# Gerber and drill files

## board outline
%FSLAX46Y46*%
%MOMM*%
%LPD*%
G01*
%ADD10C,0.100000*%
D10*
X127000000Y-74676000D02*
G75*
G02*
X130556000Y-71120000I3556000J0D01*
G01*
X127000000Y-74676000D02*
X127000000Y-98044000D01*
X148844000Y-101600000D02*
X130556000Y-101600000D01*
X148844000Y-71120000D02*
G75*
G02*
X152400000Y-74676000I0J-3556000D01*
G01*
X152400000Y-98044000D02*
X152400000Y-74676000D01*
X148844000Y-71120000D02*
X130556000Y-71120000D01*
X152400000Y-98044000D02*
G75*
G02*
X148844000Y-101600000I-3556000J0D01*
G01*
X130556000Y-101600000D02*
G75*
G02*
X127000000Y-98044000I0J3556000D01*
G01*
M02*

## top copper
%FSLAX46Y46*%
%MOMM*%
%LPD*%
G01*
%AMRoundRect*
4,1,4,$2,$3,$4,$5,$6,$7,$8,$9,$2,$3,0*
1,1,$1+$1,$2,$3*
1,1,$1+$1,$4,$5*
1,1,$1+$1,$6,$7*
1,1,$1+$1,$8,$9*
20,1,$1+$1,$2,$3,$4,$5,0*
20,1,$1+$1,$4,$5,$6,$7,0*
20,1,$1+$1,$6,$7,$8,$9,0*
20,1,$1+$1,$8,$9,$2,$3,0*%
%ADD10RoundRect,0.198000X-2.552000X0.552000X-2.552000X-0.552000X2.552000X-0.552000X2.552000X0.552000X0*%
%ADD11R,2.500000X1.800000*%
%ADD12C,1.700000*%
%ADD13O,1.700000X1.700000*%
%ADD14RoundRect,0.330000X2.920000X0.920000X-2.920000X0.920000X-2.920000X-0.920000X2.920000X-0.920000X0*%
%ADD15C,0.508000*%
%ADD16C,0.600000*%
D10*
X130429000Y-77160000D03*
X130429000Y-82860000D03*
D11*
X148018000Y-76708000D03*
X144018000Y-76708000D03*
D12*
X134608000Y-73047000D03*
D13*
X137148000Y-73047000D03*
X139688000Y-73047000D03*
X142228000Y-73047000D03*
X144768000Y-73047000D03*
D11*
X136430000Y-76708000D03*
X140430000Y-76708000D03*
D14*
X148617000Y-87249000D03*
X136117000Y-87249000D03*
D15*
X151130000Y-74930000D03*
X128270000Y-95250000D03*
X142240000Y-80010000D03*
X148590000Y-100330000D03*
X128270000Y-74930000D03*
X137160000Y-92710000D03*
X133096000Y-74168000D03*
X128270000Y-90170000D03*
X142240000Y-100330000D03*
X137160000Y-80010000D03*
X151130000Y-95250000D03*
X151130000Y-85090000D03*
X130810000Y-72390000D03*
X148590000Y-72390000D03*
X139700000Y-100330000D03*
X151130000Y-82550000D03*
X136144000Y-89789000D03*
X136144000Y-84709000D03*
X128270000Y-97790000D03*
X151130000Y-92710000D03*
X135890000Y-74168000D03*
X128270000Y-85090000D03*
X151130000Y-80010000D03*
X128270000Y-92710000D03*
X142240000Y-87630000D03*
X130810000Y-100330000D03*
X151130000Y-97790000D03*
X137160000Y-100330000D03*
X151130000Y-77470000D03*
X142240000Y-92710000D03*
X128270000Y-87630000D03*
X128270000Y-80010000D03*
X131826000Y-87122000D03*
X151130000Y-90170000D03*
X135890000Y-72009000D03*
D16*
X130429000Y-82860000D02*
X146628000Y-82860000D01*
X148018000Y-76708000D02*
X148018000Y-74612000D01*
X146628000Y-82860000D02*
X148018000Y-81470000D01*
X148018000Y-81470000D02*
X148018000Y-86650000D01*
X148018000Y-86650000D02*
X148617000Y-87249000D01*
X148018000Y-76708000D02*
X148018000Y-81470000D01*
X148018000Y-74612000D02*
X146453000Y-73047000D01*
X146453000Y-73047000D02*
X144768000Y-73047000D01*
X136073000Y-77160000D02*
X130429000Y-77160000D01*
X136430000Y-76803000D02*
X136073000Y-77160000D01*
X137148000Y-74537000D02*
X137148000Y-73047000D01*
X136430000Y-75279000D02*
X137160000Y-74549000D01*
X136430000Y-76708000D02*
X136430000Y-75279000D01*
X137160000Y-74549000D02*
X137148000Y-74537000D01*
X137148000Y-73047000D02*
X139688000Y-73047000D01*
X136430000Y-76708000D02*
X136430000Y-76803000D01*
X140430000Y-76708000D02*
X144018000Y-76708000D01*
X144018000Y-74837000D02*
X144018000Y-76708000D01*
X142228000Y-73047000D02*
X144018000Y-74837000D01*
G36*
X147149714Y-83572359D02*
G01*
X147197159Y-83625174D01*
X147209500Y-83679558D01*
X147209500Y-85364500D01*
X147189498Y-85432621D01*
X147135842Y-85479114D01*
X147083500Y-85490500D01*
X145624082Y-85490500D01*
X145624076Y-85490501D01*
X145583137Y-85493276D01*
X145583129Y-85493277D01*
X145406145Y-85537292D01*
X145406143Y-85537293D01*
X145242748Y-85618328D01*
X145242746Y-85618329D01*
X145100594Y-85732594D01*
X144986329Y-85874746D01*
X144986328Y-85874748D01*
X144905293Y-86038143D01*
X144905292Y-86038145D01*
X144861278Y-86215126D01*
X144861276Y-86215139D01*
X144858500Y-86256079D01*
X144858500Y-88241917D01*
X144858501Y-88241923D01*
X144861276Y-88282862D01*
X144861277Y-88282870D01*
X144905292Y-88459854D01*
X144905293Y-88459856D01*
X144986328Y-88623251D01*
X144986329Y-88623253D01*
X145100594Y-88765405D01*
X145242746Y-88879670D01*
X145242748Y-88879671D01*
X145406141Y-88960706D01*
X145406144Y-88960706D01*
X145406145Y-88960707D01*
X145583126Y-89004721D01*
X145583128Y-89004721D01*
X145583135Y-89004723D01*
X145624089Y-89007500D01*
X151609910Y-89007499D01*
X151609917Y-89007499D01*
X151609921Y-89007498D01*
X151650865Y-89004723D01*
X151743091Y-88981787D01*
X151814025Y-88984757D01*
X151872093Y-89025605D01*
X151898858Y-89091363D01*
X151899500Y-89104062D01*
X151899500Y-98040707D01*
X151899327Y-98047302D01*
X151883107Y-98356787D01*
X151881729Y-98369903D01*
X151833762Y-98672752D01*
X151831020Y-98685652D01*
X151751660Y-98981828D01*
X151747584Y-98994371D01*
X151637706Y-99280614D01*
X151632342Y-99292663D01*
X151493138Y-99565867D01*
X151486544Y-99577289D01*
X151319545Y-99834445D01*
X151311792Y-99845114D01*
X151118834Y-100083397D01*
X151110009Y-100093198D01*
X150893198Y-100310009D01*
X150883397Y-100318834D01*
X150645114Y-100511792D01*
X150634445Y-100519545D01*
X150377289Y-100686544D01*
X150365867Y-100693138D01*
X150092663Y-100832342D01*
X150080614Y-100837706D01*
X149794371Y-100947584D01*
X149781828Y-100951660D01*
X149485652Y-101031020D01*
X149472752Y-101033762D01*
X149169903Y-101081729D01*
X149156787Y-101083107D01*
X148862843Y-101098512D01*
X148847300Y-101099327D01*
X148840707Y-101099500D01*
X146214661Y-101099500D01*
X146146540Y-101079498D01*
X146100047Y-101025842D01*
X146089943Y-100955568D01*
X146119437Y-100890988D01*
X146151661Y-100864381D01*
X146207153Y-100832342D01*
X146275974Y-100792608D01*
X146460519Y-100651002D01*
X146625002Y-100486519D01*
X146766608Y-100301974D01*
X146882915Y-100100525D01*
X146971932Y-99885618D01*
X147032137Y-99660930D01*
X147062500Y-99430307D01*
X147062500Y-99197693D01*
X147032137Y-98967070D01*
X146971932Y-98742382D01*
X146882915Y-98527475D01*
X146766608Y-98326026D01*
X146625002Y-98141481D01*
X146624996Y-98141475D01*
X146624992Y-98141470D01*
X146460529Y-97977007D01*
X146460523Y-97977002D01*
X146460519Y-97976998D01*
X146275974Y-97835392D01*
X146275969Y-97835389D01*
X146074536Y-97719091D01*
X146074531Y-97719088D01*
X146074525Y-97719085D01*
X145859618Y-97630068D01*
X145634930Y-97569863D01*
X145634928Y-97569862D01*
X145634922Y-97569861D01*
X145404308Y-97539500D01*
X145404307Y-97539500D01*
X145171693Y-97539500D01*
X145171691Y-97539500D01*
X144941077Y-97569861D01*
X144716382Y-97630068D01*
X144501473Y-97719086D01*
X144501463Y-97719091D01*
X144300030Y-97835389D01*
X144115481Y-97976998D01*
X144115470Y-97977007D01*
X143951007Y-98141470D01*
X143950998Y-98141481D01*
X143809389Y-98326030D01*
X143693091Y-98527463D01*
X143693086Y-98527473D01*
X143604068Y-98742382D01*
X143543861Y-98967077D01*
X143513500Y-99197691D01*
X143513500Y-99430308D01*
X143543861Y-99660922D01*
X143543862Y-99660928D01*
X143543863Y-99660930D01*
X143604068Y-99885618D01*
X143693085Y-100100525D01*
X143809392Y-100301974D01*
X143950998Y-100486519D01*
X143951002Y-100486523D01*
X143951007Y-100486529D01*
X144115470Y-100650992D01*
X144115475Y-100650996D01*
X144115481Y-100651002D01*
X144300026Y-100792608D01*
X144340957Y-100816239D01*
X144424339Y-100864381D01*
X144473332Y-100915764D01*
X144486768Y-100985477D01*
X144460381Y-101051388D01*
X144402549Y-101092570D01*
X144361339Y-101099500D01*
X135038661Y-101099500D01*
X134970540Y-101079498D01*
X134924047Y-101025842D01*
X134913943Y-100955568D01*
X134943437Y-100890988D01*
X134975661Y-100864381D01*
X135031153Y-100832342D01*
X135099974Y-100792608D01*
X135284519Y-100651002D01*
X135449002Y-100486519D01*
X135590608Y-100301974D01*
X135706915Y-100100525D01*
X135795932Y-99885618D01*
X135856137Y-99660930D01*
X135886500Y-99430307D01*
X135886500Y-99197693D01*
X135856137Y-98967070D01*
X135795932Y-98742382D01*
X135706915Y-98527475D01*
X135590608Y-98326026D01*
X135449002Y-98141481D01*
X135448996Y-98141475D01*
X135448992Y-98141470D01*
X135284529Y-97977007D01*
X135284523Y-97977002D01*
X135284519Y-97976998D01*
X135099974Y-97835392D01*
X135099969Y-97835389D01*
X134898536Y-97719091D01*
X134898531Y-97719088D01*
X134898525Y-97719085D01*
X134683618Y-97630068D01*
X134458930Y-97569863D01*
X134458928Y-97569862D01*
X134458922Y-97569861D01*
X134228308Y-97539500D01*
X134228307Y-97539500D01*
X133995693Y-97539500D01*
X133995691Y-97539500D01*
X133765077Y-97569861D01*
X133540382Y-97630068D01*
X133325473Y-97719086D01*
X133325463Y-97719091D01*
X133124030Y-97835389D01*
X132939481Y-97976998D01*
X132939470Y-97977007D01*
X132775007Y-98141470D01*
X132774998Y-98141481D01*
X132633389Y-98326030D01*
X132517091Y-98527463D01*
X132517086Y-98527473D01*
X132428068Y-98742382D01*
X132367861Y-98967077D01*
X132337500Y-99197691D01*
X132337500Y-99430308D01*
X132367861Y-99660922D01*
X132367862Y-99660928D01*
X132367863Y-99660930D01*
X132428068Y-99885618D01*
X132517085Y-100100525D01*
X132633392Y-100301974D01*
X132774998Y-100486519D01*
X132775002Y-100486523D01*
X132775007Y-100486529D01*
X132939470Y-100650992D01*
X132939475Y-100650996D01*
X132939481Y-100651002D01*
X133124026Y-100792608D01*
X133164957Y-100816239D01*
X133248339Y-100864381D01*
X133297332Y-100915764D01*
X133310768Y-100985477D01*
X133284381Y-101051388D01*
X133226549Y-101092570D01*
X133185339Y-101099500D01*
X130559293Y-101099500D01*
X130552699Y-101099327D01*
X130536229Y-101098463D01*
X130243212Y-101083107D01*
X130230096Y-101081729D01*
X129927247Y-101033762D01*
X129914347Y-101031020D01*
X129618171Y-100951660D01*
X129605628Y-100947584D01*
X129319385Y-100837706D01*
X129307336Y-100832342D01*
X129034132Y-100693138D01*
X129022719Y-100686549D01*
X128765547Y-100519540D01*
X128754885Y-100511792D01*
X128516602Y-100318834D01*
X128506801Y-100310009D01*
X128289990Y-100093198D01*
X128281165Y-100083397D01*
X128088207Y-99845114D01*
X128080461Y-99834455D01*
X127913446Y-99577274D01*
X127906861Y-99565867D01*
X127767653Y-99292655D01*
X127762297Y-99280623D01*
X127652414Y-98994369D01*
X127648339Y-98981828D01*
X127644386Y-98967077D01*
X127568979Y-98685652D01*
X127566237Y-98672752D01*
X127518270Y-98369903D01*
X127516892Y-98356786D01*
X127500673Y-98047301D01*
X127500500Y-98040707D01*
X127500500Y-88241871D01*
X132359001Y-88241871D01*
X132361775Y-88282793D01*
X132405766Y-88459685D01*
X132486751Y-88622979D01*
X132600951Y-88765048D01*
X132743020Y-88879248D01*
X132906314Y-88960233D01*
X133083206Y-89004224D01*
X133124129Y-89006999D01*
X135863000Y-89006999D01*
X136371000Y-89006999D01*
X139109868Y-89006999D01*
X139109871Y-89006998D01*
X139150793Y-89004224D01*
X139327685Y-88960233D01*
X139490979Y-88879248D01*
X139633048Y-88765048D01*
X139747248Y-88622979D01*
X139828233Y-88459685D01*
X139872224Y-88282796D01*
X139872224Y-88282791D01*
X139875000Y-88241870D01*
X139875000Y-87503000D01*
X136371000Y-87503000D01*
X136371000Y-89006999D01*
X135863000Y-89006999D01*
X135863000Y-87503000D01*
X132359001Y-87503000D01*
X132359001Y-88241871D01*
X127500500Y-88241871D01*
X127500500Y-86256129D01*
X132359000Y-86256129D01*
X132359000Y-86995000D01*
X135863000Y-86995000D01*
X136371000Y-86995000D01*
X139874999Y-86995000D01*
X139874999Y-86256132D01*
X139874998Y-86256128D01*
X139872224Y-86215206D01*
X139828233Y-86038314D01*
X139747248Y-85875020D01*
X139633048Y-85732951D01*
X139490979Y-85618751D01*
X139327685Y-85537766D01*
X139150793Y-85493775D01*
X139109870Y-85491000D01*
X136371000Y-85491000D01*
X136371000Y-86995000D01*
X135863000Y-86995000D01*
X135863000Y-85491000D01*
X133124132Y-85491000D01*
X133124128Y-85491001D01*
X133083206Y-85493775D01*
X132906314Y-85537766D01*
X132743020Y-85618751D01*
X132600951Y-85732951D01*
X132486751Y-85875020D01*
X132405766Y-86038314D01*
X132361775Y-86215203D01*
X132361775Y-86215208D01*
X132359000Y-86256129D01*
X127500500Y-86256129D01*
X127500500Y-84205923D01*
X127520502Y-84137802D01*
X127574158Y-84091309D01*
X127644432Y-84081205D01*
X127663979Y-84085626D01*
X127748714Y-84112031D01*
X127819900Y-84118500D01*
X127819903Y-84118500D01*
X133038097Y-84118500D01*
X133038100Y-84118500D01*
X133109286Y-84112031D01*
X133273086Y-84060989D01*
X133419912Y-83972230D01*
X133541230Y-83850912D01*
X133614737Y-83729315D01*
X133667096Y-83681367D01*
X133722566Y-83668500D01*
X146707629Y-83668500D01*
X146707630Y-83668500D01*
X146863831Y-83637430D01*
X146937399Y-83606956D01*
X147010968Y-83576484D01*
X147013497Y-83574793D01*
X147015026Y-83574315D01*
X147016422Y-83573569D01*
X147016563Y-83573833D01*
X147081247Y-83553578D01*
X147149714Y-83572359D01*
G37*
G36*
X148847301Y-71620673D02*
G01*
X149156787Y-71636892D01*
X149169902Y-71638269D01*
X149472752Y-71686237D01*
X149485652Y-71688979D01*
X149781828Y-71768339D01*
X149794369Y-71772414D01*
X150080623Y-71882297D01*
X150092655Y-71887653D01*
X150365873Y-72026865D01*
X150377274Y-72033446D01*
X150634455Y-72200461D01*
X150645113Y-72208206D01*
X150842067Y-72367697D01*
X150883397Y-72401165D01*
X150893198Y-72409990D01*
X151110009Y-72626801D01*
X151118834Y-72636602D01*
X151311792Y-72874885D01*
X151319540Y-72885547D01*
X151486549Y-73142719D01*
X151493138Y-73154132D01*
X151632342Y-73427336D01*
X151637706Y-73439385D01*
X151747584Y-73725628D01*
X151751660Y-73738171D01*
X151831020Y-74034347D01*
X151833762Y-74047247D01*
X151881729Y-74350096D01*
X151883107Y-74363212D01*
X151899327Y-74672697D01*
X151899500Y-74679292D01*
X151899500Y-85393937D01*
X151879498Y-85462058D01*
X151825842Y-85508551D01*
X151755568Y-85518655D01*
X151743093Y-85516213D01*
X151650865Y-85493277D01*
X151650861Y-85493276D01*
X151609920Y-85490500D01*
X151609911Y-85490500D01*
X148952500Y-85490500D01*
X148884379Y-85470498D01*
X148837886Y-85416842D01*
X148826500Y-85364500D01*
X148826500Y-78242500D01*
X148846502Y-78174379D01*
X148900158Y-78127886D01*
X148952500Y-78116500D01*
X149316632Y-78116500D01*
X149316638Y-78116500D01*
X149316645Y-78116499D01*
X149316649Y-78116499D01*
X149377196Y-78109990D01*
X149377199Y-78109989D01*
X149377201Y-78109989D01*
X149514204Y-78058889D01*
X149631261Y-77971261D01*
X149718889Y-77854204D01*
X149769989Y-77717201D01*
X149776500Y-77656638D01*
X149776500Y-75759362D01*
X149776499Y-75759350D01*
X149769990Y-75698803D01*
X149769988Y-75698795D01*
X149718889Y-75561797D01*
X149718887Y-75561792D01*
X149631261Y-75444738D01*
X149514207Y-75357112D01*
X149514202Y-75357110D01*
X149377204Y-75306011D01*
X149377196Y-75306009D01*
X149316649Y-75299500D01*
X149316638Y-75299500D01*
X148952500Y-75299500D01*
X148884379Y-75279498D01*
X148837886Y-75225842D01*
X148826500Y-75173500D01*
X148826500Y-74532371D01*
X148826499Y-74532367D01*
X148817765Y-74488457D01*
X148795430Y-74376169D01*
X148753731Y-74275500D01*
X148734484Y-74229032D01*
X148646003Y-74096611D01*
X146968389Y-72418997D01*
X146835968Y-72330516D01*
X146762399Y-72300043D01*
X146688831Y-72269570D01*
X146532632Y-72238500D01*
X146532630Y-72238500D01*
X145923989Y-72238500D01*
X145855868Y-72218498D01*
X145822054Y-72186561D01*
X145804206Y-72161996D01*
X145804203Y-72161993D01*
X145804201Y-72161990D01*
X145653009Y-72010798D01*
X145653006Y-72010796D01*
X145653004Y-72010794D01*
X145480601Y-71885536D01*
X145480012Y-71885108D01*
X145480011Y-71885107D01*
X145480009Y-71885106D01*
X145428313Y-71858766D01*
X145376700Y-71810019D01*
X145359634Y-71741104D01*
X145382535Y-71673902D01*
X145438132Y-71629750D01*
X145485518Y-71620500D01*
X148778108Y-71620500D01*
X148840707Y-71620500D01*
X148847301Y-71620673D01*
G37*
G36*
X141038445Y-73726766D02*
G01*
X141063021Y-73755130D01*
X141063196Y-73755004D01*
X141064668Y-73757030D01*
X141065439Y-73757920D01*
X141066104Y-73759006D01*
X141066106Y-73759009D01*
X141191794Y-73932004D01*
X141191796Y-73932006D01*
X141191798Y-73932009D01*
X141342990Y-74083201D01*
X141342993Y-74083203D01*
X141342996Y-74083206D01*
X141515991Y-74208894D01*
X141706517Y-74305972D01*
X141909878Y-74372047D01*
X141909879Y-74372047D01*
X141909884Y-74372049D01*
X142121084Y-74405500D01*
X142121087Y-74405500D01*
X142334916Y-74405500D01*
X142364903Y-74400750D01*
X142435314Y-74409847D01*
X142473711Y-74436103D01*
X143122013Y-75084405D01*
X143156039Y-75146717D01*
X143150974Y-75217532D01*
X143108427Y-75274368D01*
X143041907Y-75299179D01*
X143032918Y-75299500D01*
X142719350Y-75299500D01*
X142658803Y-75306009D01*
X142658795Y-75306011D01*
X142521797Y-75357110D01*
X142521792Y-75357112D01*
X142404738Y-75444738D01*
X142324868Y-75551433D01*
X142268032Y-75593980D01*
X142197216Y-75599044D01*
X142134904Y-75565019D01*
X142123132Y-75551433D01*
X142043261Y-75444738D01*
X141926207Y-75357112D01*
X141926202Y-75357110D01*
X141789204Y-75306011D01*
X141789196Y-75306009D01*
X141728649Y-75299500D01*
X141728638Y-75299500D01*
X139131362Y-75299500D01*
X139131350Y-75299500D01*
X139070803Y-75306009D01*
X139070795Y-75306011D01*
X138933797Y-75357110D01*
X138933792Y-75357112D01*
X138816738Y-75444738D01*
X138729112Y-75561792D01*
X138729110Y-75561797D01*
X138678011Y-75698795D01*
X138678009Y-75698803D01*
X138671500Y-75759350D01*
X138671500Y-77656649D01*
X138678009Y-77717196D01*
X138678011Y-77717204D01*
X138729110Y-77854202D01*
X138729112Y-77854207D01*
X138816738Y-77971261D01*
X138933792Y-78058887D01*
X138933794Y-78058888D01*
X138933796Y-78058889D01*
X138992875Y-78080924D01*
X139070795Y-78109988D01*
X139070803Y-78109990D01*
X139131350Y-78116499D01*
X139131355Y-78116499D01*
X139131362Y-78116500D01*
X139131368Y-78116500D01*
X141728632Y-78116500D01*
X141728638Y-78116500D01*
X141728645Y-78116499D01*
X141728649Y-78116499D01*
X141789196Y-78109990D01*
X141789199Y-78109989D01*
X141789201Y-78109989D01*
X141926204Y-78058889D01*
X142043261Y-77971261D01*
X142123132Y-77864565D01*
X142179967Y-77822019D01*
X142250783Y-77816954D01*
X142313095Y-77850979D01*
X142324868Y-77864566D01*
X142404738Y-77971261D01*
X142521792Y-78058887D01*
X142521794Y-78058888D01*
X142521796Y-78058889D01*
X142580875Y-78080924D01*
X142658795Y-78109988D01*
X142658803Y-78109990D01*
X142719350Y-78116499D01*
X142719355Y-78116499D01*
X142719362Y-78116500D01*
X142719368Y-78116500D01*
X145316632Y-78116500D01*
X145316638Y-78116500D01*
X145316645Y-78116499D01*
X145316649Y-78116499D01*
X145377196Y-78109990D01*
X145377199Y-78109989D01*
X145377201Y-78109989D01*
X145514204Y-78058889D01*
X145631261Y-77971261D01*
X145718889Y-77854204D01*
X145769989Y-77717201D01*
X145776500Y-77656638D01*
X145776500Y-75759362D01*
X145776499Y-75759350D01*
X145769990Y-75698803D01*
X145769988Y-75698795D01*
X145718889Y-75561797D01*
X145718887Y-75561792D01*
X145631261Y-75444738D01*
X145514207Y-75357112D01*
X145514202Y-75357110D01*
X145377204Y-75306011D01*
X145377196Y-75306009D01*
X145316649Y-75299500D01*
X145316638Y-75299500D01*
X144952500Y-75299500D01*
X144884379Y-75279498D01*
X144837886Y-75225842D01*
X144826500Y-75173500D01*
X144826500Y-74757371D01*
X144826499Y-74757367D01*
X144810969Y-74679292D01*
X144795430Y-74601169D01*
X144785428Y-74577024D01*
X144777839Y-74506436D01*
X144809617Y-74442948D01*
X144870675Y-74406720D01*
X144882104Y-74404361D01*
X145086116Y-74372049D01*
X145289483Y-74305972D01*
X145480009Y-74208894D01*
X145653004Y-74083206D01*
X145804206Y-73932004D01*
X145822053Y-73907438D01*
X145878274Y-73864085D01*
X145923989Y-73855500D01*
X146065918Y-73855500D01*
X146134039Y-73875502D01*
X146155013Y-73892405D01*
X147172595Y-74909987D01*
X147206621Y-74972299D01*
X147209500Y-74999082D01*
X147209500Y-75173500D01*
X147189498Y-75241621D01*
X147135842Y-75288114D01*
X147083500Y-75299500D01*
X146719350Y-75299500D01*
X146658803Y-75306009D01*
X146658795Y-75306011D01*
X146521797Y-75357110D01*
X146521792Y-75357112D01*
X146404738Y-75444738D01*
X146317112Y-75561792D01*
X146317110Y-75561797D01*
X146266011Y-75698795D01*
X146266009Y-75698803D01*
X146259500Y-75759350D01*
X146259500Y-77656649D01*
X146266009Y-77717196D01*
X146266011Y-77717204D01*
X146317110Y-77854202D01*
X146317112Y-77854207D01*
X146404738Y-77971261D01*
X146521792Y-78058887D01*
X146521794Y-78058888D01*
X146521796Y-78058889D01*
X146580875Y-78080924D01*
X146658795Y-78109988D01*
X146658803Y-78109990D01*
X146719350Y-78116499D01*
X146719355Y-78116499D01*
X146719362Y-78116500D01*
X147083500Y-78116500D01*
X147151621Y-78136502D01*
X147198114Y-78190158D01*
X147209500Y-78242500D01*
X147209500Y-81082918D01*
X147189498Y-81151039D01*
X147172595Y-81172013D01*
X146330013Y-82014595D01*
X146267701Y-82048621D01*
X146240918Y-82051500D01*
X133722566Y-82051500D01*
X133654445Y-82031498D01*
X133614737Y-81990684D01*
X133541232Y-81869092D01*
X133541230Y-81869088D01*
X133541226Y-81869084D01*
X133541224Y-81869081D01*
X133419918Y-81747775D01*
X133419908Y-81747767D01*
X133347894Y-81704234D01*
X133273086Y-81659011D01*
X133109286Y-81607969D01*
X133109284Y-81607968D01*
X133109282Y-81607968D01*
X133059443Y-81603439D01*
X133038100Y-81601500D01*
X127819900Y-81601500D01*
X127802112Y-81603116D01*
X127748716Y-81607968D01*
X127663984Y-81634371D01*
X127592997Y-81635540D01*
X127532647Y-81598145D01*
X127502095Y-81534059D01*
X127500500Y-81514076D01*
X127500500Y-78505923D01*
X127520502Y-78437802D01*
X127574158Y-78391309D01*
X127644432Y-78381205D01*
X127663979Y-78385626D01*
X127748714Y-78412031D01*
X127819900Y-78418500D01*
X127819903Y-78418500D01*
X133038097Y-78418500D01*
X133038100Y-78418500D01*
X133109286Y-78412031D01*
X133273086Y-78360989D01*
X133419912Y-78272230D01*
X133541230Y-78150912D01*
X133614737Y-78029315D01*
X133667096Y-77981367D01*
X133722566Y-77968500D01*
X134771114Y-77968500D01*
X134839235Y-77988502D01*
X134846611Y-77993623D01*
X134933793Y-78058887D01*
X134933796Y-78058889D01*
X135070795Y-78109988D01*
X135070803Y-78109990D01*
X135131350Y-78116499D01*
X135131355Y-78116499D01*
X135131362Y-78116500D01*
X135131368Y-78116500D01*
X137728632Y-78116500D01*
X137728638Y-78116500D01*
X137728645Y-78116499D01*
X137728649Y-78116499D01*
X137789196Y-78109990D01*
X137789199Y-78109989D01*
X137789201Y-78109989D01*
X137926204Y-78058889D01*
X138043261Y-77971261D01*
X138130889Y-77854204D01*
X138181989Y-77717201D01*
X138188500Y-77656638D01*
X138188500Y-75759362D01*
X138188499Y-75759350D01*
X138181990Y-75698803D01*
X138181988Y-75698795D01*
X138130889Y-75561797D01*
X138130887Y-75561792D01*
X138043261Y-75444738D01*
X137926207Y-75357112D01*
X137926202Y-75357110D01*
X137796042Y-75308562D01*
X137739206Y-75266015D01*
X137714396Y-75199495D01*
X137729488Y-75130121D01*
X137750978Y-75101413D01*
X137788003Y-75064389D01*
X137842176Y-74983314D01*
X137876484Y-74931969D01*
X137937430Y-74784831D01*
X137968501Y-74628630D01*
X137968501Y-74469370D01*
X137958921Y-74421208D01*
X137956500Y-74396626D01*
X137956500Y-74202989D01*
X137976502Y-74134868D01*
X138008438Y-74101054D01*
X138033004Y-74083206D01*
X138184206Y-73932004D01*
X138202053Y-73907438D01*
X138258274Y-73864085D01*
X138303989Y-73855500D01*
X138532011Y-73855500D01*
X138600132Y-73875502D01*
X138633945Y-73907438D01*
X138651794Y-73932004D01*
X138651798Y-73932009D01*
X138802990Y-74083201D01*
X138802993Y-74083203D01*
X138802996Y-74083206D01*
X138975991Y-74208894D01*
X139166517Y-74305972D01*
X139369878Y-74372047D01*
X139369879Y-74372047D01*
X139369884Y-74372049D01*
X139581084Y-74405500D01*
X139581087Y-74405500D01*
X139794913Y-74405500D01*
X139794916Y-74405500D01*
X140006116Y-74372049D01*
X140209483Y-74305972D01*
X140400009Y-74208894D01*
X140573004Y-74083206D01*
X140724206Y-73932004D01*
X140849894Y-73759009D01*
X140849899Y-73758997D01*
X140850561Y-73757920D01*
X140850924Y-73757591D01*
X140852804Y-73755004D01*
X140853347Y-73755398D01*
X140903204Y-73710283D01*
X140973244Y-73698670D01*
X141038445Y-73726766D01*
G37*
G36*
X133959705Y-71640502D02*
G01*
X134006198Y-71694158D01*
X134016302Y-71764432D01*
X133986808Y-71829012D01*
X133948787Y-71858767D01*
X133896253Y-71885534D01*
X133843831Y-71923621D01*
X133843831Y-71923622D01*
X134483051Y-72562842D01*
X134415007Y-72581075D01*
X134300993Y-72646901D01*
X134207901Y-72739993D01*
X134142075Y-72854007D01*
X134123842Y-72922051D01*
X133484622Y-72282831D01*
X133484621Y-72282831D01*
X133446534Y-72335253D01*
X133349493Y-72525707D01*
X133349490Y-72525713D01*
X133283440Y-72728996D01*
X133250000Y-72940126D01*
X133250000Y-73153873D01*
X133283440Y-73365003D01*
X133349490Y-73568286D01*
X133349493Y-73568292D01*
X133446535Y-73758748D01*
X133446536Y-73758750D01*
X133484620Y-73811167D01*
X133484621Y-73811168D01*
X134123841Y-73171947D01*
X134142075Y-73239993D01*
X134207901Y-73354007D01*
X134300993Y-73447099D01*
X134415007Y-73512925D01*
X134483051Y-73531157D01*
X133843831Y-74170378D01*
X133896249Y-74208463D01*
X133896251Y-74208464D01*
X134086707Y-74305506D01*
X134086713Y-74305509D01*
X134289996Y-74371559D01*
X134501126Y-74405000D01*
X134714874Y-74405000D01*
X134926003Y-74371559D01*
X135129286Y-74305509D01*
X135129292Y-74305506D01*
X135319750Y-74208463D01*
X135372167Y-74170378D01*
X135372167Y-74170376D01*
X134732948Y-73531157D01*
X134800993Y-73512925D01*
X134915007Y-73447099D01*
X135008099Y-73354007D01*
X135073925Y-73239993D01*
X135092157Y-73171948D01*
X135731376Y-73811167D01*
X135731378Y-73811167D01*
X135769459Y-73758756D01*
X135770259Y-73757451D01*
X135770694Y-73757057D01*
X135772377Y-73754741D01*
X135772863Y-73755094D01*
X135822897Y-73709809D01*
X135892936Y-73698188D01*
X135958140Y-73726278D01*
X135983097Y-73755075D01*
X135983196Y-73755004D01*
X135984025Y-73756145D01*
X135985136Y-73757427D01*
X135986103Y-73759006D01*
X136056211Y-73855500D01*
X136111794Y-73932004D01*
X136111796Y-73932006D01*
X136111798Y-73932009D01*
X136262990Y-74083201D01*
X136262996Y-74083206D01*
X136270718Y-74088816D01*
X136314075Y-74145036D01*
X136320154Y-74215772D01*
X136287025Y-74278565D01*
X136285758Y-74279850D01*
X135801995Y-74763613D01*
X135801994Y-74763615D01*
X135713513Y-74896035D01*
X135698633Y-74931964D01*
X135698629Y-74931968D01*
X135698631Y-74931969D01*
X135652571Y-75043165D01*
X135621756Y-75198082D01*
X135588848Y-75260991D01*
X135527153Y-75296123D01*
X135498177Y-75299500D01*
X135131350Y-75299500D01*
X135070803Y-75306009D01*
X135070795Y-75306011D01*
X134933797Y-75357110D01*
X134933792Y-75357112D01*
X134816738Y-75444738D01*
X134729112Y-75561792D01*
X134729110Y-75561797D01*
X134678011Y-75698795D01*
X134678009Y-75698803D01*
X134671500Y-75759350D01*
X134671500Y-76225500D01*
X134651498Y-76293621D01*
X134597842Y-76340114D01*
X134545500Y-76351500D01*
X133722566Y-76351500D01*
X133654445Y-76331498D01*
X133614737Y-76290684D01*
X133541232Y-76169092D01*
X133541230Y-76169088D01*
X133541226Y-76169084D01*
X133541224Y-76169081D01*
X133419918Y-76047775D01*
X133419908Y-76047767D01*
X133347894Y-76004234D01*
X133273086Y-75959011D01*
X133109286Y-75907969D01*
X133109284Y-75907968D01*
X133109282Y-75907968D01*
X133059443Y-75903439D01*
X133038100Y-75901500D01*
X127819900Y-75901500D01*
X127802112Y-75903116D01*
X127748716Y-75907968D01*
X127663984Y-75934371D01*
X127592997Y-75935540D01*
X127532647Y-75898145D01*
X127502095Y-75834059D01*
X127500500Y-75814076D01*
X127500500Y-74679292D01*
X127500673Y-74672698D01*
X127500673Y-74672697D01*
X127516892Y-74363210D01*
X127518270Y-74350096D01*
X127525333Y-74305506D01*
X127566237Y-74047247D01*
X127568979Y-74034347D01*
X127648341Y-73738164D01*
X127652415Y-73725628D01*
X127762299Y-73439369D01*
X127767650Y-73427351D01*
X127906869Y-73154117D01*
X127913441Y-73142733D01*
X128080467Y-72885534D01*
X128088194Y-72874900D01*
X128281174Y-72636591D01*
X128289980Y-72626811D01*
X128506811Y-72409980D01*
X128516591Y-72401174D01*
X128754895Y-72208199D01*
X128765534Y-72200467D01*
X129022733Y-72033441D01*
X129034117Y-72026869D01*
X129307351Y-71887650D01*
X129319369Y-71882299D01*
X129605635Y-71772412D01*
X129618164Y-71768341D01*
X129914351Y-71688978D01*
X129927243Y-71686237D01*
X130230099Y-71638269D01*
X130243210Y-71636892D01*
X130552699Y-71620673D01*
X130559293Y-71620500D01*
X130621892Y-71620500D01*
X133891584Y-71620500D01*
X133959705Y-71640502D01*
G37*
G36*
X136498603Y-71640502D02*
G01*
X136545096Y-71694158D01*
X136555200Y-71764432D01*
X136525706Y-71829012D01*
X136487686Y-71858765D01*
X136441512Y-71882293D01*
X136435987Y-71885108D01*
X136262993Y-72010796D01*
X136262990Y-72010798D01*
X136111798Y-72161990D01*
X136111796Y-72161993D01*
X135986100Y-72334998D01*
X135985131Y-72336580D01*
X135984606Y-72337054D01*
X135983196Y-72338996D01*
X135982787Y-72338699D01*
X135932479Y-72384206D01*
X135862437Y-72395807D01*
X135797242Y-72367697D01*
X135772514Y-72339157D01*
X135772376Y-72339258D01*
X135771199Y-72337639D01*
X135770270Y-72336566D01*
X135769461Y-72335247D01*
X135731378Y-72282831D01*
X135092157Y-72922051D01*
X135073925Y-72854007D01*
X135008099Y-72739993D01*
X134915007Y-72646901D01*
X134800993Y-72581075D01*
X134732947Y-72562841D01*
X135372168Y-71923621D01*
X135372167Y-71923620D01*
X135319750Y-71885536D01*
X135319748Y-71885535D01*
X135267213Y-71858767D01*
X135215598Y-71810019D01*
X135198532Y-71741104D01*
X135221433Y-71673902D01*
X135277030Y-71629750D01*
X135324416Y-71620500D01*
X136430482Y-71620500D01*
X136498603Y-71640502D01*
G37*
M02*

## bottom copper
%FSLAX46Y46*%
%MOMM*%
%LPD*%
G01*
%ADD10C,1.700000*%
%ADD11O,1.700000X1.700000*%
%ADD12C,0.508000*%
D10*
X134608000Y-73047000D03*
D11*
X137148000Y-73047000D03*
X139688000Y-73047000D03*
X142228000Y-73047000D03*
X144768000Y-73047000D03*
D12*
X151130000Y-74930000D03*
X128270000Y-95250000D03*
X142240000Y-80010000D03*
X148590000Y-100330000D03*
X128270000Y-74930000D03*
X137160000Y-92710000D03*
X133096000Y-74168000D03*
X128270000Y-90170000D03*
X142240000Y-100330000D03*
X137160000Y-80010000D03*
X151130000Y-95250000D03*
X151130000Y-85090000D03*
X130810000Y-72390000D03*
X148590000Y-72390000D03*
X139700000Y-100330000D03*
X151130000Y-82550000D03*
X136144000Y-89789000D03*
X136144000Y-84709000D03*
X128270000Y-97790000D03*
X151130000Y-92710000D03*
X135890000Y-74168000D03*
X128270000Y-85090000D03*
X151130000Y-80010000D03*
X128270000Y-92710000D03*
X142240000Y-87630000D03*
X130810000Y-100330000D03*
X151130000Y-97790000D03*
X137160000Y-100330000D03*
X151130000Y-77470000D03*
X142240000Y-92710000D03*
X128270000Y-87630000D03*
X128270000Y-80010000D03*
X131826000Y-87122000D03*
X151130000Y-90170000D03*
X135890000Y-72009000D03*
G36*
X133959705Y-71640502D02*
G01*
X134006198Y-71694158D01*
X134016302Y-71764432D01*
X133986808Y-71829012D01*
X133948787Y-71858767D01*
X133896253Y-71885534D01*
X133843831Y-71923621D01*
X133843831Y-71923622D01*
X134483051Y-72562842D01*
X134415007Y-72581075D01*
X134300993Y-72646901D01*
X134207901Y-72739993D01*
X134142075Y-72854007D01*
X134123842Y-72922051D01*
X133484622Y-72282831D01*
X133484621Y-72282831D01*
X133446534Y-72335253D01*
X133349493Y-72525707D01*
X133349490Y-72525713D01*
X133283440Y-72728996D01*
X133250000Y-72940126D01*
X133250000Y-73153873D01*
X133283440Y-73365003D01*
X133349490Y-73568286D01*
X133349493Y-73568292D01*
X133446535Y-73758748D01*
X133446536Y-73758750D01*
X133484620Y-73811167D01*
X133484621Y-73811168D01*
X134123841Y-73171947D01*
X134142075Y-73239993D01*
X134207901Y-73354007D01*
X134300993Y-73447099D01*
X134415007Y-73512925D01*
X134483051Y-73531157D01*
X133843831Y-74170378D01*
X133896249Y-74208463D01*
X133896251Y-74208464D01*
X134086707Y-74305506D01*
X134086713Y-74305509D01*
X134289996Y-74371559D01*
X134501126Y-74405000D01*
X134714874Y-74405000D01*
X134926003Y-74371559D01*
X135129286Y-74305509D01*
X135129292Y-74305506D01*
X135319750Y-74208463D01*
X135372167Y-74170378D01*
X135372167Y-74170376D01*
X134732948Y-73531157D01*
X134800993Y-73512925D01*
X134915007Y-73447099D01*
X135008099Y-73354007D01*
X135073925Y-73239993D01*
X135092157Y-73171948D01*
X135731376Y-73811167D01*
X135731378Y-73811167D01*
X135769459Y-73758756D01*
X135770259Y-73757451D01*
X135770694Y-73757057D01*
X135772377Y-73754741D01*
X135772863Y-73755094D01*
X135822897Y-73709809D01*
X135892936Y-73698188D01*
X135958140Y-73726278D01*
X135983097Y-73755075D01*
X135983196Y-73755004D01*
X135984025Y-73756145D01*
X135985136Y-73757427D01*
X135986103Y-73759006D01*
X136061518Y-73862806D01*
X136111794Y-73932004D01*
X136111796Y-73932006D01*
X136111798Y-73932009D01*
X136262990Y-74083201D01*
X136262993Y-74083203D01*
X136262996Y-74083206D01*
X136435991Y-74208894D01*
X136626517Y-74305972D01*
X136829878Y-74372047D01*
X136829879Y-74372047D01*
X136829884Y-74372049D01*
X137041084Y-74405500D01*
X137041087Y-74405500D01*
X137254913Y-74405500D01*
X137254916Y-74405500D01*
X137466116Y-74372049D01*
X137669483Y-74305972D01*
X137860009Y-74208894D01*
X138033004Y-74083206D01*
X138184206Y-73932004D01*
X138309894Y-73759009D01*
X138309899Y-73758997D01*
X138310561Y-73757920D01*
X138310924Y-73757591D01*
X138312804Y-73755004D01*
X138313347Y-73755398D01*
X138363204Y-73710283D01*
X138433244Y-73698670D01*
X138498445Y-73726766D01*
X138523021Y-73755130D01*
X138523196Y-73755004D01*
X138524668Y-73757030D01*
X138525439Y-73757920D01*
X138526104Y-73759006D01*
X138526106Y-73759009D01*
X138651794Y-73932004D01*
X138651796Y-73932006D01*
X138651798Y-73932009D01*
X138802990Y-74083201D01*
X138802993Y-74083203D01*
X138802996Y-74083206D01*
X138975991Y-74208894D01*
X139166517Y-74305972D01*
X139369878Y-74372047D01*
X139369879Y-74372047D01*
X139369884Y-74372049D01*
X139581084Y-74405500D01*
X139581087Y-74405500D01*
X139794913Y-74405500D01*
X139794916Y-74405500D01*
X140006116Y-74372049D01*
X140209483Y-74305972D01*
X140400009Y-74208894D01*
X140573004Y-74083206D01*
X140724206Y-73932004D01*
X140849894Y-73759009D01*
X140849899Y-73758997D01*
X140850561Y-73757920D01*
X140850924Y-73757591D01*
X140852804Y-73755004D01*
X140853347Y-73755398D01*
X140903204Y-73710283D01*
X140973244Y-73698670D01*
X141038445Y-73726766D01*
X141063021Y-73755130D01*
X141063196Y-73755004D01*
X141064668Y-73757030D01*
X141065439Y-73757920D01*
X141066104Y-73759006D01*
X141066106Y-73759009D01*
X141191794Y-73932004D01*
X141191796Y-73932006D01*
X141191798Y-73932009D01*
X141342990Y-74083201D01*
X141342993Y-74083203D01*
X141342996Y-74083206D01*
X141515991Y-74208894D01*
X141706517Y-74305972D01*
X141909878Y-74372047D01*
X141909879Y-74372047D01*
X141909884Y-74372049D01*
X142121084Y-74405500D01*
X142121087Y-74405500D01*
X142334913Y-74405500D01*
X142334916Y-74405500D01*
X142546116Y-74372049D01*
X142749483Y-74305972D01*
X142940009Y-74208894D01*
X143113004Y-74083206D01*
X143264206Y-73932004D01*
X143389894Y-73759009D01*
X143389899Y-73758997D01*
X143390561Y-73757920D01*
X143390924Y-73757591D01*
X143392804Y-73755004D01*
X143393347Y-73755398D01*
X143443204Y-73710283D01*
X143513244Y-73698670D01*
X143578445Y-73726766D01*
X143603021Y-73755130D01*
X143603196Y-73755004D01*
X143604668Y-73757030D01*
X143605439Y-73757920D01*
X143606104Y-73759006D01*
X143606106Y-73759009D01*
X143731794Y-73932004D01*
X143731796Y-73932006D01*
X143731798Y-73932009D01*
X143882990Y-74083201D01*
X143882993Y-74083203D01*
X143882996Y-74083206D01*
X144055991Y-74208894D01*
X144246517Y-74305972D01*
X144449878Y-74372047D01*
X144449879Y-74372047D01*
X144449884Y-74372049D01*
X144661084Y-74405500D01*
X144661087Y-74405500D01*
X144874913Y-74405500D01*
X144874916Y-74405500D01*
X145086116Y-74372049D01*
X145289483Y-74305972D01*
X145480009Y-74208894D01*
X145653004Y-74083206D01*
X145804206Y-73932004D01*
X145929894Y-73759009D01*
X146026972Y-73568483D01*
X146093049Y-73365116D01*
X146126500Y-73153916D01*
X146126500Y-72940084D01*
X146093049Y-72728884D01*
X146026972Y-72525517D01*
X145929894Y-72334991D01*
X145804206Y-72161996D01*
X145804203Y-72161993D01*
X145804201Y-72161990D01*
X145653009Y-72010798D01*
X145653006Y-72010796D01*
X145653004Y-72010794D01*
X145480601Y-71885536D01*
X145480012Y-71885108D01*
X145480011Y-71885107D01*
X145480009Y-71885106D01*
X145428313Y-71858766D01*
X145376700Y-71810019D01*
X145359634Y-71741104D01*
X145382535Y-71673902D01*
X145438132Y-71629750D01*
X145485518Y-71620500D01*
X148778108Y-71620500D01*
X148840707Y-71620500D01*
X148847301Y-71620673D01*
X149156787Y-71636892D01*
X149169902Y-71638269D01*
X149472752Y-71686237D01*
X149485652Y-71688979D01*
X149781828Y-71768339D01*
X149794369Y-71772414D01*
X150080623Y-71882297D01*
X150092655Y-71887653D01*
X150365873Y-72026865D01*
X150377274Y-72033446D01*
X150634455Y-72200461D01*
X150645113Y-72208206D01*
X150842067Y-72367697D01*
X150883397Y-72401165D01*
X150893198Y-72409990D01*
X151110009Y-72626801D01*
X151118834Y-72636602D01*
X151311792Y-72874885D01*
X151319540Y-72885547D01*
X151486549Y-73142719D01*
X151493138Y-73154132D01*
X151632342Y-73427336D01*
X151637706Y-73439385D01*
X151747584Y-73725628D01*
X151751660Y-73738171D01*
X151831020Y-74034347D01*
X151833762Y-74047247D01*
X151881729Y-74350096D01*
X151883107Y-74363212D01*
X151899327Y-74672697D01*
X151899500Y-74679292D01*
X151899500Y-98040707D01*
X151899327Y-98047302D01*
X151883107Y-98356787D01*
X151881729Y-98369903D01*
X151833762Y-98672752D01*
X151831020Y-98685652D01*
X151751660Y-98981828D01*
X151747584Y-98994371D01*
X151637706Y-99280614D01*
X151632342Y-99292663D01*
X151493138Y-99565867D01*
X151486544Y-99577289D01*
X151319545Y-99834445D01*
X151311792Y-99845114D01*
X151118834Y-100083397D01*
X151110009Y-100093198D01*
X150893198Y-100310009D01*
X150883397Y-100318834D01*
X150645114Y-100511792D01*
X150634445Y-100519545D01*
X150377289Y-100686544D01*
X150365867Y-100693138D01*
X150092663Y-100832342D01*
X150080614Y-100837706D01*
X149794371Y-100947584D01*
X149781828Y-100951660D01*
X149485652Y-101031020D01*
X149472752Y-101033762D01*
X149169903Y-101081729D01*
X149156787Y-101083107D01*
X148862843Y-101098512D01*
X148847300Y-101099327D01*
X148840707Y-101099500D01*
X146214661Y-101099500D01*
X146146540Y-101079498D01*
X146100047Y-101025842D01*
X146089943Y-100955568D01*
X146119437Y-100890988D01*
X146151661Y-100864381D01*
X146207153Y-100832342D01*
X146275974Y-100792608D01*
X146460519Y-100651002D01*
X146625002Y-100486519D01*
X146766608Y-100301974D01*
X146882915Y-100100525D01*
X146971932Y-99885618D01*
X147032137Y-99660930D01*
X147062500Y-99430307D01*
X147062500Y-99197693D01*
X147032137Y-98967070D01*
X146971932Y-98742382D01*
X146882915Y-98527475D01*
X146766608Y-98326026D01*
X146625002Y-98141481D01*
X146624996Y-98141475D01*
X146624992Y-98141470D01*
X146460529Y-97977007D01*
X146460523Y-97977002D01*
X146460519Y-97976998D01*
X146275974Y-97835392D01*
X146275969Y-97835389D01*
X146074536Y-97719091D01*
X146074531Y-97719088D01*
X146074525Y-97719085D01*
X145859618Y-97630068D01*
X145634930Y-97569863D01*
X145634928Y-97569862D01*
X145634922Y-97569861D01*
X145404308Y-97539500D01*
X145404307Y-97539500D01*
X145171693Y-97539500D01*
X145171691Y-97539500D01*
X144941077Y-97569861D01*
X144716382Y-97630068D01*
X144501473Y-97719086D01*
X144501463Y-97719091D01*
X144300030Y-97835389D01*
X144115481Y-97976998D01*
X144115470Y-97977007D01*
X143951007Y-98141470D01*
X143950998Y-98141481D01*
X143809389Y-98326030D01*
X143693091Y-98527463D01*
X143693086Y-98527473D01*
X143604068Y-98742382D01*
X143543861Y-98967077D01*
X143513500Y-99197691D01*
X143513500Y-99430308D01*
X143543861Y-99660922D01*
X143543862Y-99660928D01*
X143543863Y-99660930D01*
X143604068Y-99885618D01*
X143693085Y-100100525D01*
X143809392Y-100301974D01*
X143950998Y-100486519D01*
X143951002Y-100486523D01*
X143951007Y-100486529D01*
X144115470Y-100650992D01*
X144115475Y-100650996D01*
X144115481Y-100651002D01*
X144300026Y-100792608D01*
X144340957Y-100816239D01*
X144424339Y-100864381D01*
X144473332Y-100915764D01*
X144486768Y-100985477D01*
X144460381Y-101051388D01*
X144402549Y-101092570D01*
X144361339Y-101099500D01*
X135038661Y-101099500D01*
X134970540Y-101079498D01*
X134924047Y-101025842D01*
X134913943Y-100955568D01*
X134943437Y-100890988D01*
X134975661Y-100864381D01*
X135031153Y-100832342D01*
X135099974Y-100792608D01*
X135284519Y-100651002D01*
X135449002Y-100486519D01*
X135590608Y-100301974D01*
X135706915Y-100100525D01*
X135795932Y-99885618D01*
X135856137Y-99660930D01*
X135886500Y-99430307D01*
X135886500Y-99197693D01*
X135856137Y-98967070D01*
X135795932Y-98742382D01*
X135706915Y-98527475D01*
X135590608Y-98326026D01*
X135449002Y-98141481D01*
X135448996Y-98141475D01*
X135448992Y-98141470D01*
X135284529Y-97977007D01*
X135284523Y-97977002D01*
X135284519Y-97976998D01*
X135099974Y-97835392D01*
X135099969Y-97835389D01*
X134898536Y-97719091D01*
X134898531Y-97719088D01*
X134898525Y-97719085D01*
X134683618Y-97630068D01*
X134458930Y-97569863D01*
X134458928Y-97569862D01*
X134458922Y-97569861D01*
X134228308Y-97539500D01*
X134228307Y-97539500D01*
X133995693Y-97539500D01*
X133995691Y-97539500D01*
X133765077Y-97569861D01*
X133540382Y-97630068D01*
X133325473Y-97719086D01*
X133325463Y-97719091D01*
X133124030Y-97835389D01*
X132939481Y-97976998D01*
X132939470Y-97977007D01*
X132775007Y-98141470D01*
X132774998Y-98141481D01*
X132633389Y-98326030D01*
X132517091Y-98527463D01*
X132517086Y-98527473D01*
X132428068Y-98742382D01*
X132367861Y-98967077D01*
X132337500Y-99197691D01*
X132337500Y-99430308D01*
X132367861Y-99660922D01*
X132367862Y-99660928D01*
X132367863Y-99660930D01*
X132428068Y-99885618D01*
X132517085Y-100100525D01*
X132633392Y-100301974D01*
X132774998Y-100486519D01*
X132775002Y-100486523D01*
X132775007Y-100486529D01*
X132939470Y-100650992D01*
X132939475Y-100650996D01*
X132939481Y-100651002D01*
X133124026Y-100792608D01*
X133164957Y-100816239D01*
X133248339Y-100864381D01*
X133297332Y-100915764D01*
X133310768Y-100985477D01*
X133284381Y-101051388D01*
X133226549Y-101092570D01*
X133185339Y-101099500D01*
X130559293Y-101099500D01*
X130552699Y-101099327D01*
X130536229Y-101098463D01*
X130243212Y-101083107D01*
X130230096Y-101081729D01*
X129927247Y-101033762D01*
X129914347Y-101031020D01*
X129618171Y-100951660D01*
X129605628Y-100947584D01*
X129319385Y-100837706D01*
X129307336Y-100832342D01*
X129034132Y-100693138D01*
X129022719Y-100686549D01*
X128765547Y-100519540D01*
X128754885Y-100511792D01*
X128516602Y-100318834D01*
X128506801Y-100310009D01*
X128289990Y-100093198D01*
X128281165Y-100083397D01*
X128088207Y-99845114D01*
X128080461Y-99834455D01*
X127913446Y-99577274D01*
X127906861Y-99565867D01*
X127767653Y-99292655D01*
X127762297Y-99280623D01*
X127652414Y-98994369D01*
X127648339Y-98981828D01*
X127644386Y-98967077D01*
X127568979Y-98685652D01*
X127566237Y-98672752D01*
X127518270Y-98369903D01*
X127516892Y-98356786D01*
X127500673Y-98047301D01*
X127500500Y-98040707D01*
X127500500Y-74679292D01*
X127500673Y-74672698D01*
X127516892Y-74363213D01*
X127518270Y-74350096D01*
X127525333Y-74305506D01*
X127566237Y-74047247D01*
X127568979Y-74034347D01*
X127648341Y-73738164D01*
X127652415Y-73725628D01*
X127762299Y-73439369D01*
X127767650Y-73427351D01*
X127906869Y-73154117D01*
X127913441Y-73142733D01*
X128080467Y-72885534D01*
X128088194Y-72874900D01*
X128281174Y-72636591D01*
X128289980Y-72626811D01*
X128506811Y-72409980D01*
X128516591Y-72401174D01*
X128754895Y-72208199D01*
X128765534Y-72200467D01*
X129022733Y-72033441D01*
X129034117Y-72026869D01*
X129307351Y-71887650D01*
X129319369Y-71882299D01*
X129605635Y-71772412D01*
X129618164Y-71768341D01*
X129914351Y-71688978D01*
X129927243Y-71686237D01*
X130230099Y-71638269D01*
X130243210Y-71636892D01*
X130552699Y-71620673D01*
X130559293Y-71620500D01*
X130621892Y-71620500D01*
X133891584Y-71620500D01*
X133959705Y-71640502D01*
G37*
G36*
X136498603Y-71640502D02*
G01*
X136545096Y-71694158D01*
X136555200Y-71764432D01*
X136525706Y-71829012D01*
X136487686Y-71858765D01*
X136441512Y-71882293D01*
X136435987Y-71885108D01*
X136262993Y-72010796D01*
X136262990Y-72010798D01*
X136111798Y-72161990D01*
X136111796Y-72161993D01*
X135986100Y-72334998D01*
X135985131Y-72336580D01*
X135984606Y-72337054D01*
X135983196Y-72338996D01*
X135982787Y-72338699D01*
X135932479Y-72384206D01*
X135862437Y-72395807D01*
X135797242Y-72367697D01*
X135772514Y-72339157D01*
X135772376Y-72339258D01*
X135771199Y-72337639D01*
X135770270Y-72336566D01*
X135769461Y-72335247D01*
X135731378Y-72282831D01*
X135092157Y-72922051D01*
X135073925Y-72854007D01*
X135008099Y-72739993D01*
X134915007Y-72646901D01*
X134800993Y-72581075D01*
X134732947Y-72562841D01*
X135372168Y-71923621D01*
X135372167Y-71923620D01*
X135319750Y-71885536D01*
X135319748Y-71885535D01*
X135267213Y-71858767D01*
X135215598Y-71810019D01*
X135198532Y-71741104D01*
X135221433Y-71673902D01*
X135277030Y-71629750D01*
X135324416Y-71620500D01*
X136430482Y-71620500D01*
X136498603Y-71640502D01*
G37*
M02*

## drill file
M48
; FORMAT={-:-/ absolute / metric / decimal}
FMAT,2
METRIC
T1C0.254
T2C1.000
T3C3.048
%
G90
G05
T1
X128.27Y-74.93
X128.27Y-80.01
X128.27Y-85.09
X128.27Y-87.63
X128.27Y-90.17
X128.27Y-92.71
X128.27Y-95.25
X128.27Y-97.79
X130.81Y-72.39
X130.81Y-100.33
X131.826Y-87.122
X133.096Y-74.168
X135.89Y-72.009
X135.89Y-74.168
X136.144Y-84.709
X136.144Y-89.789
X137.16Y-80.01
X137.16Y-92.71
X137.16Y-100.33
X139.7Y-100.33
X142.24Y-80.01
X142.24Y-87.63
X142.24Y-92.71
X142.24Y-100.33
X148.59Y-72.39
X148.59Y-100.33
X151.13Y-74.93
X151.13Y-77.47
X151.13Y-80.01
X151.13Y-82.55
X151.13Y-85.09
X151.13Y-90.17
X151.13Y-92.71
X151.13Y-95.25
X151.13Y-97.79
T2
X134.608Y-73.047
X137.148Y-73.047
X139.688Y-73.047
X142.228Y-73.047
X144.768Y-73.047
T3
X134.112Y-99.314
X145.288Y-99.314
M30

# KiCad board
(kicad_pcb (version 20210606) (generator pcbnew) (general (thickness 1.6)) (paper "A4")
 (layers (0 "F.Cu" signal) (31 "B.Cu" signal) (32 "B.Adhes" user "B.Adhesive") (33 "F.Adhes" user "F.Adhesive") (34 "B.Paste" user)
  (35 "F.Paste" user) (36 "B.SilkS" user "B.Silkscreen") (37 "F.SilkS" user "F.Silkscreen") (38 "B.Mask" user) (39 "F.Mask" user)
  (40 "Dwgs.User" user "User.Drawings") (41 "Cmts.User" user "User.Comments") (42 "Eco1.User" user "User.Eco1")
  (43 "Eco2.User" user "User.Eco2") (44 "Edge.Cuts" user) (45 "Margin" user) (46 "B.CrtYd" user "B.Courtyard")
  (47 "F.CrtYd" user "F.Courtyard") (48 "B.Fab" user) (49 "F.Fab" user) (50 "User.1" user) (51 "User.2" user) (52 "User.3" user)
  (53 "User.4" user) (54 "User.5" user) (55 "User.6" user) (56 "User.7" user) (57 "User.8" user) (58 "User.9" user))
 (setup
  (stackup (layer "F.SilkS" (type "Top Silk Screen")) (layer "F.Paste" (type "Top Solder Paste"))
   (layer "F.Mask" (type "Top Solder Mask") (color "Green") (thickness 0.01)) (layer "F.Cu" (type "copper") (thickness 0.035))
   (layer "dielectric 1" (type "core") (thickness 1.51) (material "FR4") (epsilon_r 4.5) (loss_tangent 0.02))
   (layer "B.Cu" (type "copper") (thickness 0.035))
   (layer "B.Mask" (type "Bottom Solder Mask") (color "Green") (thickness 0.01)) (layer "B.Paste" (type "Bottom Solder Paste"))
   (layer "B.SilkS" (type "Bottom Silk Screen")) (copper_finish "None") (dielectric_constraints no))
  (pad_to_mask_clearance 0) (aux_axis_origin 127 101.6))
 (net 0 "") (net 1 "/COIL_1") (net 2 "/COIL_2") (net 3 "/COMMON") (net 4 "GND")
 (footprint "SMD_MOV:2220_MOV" (layer "F.Cu") (at 130.429 80.01 -90)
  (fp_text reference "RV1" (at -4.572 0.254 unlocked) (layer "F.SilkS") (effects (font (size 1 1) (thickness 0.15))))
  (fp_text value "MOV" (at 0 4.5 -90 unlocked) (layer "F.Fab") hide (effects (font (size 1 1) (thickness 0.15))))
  (pad "1" smd roundrect locked (at -2.85 0 270) (size 1.5 5.5) (layers "F.Cu" "F.Paste" "F.Mask") (roundrect_rratio 0.132)
   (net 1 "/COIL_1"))
  (pad "2" smd roundrect locked (at 2.85 0 270) (size 1.5 5.5) (layers "F.Cu" "F.Paste" "F.Mask") (roundrect_rratio 0.132) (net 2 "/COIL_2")))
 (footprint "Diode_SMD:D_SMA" (layer "F.Cu") (at 146.018 76.708 180)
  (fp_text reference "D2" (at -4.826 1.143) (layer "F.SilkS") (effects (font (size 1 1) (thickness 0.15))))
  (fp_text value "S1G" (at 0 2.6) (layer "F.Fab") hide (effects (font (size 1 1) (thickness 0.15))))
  (pad "1" smd rect locked (at -2 0 180) (size 2.5 1.8) (layers "F.Cu" "F.Paste" "F.Mask") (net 2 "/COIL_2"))
  (pad "2" smd rect locked (at 2 0 180) (size 2.5 1.8) (layers "F.Cu" "F.Paste" "F.Mask") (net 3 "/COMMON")))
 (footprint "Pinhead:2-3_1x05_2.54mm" (layer "F.Cu") (at 139.7 73.025 90)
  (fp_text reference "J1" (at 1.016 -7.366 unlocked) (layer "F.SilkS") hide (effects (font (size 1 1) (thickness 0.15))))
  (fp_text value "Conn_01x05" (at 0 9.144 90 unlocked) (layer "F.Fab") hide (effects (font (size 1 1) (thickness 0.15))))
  (pad "1" thru_hole circle locked (at -0.022 -5.092 90) (size 1.7 1.7) (drill 1) (layers *.Cu *.Mask) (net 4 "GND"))
  (pad "2" thru_hole oval locked (at -0.022 -2.552 90) (size 1.7 1.7) (drill 1) (layers *.Cu *.Mask) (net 1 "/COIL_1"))
  (pad "3" thru_hole oval locked (at -0.022 -0.012 90) (size 1.7 1.7) (drill 1) (layers *.Cu *.Mask) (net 1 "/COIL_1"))
  (pad "4" thru_hole oval locked (at -0.022 2.528 90) (size 1.7 1.7) (drill 1) (layers *.Cu *.Mask) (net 3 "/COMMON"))
  (pad "5" thru_hole oval locked (at -0.022 5.068 90) (size 1.7 1.7) (drill 1) (layers *.Cu *.Mask) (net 2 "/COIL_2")))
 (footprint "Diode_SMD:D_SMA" (layer "F.Cu") (at 138.43 76.708)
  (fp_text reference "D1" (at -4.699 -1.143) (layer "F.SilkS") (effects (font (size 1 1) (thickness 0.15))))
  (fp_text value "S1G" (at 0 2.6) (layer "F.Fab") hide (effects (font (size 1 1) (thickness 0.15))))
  (pad "1" smd rect locked (at -2 0) (size 2.5 1.8) (layers "F.Cu" "F.Paste" "F.Mask") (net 1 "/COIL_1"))
  (pad "2" smd rect locked (at 2 0) (size 2.5 1.8) (layers "F.Cu" "F.Paste" "F.Mask") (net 3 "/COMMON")))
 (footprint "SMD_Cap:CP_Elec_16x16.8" (layer "F.Cu") (at 142.367 87.249 180)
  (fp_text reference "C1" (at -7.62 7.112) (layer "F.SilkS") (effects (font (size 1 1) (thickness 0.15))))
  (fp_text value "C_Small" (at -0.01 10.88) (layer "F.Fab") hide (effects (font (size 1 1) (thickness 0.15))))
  (pad "1" smd roundrect locked (at -6.25 0 180) (size 6.5 2.5) (layers "F.Cu" "F.Paste" "F.Mask") (roundrect_rratio 0.132)
   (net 2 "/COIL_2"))
  (pad "2" smd roundrect locked (at 6.25 0 180) (size 6.5 2.5) (layers "F.Cu" "F.Paste" "F.Mask") (roundrect_rratio 0.132) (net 4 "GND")))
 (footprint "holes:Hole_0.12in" (layer "F.Cu") (at 145.288 99.314)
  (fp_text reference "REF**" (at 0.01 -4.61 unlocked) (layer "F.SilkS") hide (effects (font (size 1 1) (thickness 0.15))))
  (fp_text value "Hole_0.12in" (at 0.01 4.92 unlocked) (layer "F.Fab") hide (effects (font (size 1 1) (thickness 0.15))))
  (pad "" np_thru_hole circle locked (at 0 0) (size 3.048 3.048) (drill 3.048) (layers F&B.Cu *.Mask)))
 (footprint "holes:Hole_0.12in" (layer "F.Cu") (at 134.112 99.314)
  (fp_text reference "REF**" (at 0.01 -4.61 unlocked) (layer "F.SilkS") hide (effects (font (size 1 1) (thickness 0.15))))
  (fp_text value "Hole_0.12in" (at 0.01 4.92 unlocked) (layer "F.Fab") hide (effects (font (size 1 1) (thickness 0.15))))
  (pad "" np_thru_hole circle locked (at 0 0) (size 3.048 3.048) (drill 3.048) (layers F&B.Cu *.Mask)))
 (gr_arc (start 130.556 74.676) (end 130.556 71.12) (angle -90) (layer "Edge.Cuts") (width 0.1))
 (gr_line (start 127 74.676) (end 127 98.044) (layer "Edge.Cuts") (width 0.1))
 (gr_line (start 148.844 101.6) (end 130.556 101.6) (layer "Edge.Cuts") (width 0.1))
 (gr_arc (start 148.844 74.676) (end 148.844 71.12) (angle 90) (layer "Edge.Cuts") (width 0.1))
 (gr_line (start 152.4 98.044) (end 152.4 74.676) (layer "Edge.Cuts") (width 0.1))
 (gr_line (start 148.844 71.12) (end 130.556 71.12) (layer "Edge.Cuts") (width 0.1))
 (gr_arc (start 148.844 98.044) (end 148.844 101.6) (angle -90) (layer "Edge.Cuts") (width 0.1))
 (gr_arc (start 130.556 98.044) (end 130.556 101.6) (angle 90) (layer "Edge.Cuts") (width 0.1))
 (via (at 151.13 74.93) (size 0.508) (drill 0.254) (layers "F.Cu" "B.Cu") (free) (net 4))
 (via (at 128.27 95.25) (size 0.508) (drill 0.254) (layers "F.Cu" "B.Cu") (free) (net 4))
 (via (at 142.24 80.01) (size 0.508) (drill 0.254) (layers "F.Cu" "B.Cu") (free) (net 4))
 (via (at 148.59 100.33) (size 0.508) (drill 0.254) (layers "F.Cu" "B.Cu") (free) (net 4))
 (via (at 128.27 74.93) (size 0.508) (drill 0.254) (layers "F.Cu" "B.Cu") (free) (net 4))
 (via (at 137.16 92.71) (size 0.508) (drill 0.254) (layers "F.Cu" "B.Cu") (free) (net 4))
 (via (at 133.096 74.168) (size 0.508) (drill 0.254) (layers "F.Cu" "B.Cu") (free) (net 4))
 (via (at 128.27 90.17) (size 0.508) (drill 0.254) (layers "F.Cu" "B.Cu") (free) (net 4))
 (via (at 142.24 100.33) (size 0.508) (drill 0.254) (layers "F.Cu" "B.Cu") (free) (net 4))
 (via (at 137.16 80.01) (size 0.508) (drill 0.254) (layers "F.Cu" "B.Cu") (free) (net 4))
 (via (at 151.13 95.25) (size 0.508) (drill 0.254) (layers "F.Cu" "B.Cu") (free) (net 4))
 (via (at 151.13 85.09) (size 0.508) (drill 0.254) (layers "F.Cu" "B.Cu") (free) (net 4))
 (via (at 130.81 72.39) (size 0.508) (drill 0.254) (layers "F.Cu" "B.Cu") (free) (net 4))
 (via (at 148.59 72.39) (size 0.508) (drill 0.254) (layers "F.Cu" "B.Cu") (free) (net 4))
 (via (at 139.7 100.33) (size 0.508) (drill 0.254) (layers "F.Cu" "B.Cu") (free) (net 4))
 (via (at 151.13 82.55) (size 0.508) (drill 0.254) (layers "F.Cu" "B.Cu") (free) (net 4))
 (via (at 136.144 89.789) (size 0.508) (drill 0.254) (layers "F.Cu" "B.Cu") (free) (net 4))
 (via (at 136.144 84.709) (size 0.508) (drill 0.254) (layers "F.Cu" "B.Cu") (free) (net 4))
 (via (at 128.27 97.79) (size 0.508) (drill 0.254) (layers "F.Cu" "B.Cu") (free) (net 4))
 (via (at 151.13 92.71) (size 0.508) (drill 0.254) (layers "F.Cu" "B.Cu") (free) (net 4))
 (via (at 135.89 74.168) (size 0.508) (drill 0.254) (layers "F.Cu" "B.Cu") (free) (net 4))
 (via (at 128.27 85.09) (size 0.508) (drill 0.254) (layers "F.Cu" "B.Cu") (free) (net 4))
 (via (at 151.13 80.01) (size 0.508) (drill 0.254) (layers "F.Cu" "B.Cu") (free) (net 4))
 (via (at 128.27 92.71) (size 0.508) (drill 0.254) (layers "F.Cu" "B.Cu") (free) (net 4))
 (via (at 142.24 87.63) (size 0.508) (drill 0.254) (layers "F.Cu" "B.Cu") (free) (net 4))
 (via (at 130.81 100.33) (size 0.508) (drill 0.254) (layers "F.Cu" "B.Cu") (free) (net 4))
 (via (at 151.13 97.79) (size 0.508) (drill 0.254) (layers "F.Cu" "B.Cu") (free) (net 4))
 (via (at 137.16 100.33) (size 0.508) (drill 0.254) (layers "F.Cu" "B.Cu") (free) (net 4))
 (via (at 151.13 77.47) (size 0.508) (drill 0.254) (layers "F.Cu" "B.Cu") (free) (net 4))
 (via (at 142.24 92.71) (size 0.508) (drill 0.254) (layers "F.Cu" "B.Cu") (free) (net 4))
 (via (at 128.27 87.63) (size 0.508) (drill 0.254) (layers "F.Cu" "B.Cu") (free) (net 4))
 (via (at 128.27 80.01) (size 0.508) (drill 0.254) (layers "F.Cu" "B.Cu") (free) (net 4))
 (via (at 131.826 87.122) (size 0.508) (drill 0.254) (layers "F.Cu" "B.Cu") (free) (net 4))
 (via (at 151.13 90.17) (size 0.508) (drill 0.254) (layers "F.Cu" "B.Cu") (free) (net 4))
 (via (at 135.89 72.009) (size 0.508) (drill 0.254) (layers "F.Cu" "B.Cu") (free) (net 4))
 (segment (start 130.429 82.86) (end 146.628 82.86) (width 0.6) (layer "F.Cu") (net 2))
 (segment (start 148.018 76.708) (end 148.018 74.612) (width 0.6) (layer "F.Cu") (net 2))
 (segment (start 146.628 82.86) (end 148.018 81.47) (width 0.6) (layer "F.Cu") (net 2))
 (segment (start 148.018 81.47) (end 148.018 86.65) (width 0.6) (layer "F.Cu") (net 2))
 (segment (start 148.018 86.65) (end 148.617 87.249) (width 0.6) (layer "F.Cu") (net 2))
 (segment (start 148.018 76.708) (end 148.018 81.47) (width 0.6) (layer "F.Cu") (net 2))
 (segment (start 148.018 74.612) (end 146.453 73.047) (width 0.6) (layer "F.Cu") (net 2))
 (segment (start 146.453 73.047) (end 144.768 73.047) (width 0.6) (layer "F.Cu") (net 2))
 (segment (start 136.073 77.16) (end 130.429 77.16) (width 0.6) (layer "F.Cu") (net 1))
 (segment (start 136.43 76.803) (end 136.073 77.16) (width 0.6) (layer "F.Cu") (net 1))
 (segment (start 137.148 74.537) (end 137.148 73.047) (width 0.6) (layer "F.Cu") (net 1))
 (segment (start 136.43 75.279) (end 137.16 74.549) (width 0.6) (layer "F.Cu") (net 1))
 (segment (start 136.43 76.708) (end 136.43 75.279) (width 0.6) (layer "F.Cu") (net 1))
 (segment (start 137.16 74.549) (end 137.148 74.537) (width 0.6) (layer "F.Cu") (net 1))
 (segment (start 137.148 73.047) (end 139.688 73.047) (width 0.6) (layer "F.Cu") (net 1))
 (segment (start 136.43 76.708) (end 136.43 76.803) (width 0.6) (layer "F.Cu") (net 1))
 (segment (start 140.43 76.708) (end 144.018 76.708) (width 0.6) (layer "F.Cu") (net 3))
 (segment (start 144.018 74.837) (end 144.018 76.708) (width 0.6) (layer "F.Cu") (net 3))
 (segment (start 142.228 73.047) (end 144.018 74.837) (width 0.6) (layer "F.Cu") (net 3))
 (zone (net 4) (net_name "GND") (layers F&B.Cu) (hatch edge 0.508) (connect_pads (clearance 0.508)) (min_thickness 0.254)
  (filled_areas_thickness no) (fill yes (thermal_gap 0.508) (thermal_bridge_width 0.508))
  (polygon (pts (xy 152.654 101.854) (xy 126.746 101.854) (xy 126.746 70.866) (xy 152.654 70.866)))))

